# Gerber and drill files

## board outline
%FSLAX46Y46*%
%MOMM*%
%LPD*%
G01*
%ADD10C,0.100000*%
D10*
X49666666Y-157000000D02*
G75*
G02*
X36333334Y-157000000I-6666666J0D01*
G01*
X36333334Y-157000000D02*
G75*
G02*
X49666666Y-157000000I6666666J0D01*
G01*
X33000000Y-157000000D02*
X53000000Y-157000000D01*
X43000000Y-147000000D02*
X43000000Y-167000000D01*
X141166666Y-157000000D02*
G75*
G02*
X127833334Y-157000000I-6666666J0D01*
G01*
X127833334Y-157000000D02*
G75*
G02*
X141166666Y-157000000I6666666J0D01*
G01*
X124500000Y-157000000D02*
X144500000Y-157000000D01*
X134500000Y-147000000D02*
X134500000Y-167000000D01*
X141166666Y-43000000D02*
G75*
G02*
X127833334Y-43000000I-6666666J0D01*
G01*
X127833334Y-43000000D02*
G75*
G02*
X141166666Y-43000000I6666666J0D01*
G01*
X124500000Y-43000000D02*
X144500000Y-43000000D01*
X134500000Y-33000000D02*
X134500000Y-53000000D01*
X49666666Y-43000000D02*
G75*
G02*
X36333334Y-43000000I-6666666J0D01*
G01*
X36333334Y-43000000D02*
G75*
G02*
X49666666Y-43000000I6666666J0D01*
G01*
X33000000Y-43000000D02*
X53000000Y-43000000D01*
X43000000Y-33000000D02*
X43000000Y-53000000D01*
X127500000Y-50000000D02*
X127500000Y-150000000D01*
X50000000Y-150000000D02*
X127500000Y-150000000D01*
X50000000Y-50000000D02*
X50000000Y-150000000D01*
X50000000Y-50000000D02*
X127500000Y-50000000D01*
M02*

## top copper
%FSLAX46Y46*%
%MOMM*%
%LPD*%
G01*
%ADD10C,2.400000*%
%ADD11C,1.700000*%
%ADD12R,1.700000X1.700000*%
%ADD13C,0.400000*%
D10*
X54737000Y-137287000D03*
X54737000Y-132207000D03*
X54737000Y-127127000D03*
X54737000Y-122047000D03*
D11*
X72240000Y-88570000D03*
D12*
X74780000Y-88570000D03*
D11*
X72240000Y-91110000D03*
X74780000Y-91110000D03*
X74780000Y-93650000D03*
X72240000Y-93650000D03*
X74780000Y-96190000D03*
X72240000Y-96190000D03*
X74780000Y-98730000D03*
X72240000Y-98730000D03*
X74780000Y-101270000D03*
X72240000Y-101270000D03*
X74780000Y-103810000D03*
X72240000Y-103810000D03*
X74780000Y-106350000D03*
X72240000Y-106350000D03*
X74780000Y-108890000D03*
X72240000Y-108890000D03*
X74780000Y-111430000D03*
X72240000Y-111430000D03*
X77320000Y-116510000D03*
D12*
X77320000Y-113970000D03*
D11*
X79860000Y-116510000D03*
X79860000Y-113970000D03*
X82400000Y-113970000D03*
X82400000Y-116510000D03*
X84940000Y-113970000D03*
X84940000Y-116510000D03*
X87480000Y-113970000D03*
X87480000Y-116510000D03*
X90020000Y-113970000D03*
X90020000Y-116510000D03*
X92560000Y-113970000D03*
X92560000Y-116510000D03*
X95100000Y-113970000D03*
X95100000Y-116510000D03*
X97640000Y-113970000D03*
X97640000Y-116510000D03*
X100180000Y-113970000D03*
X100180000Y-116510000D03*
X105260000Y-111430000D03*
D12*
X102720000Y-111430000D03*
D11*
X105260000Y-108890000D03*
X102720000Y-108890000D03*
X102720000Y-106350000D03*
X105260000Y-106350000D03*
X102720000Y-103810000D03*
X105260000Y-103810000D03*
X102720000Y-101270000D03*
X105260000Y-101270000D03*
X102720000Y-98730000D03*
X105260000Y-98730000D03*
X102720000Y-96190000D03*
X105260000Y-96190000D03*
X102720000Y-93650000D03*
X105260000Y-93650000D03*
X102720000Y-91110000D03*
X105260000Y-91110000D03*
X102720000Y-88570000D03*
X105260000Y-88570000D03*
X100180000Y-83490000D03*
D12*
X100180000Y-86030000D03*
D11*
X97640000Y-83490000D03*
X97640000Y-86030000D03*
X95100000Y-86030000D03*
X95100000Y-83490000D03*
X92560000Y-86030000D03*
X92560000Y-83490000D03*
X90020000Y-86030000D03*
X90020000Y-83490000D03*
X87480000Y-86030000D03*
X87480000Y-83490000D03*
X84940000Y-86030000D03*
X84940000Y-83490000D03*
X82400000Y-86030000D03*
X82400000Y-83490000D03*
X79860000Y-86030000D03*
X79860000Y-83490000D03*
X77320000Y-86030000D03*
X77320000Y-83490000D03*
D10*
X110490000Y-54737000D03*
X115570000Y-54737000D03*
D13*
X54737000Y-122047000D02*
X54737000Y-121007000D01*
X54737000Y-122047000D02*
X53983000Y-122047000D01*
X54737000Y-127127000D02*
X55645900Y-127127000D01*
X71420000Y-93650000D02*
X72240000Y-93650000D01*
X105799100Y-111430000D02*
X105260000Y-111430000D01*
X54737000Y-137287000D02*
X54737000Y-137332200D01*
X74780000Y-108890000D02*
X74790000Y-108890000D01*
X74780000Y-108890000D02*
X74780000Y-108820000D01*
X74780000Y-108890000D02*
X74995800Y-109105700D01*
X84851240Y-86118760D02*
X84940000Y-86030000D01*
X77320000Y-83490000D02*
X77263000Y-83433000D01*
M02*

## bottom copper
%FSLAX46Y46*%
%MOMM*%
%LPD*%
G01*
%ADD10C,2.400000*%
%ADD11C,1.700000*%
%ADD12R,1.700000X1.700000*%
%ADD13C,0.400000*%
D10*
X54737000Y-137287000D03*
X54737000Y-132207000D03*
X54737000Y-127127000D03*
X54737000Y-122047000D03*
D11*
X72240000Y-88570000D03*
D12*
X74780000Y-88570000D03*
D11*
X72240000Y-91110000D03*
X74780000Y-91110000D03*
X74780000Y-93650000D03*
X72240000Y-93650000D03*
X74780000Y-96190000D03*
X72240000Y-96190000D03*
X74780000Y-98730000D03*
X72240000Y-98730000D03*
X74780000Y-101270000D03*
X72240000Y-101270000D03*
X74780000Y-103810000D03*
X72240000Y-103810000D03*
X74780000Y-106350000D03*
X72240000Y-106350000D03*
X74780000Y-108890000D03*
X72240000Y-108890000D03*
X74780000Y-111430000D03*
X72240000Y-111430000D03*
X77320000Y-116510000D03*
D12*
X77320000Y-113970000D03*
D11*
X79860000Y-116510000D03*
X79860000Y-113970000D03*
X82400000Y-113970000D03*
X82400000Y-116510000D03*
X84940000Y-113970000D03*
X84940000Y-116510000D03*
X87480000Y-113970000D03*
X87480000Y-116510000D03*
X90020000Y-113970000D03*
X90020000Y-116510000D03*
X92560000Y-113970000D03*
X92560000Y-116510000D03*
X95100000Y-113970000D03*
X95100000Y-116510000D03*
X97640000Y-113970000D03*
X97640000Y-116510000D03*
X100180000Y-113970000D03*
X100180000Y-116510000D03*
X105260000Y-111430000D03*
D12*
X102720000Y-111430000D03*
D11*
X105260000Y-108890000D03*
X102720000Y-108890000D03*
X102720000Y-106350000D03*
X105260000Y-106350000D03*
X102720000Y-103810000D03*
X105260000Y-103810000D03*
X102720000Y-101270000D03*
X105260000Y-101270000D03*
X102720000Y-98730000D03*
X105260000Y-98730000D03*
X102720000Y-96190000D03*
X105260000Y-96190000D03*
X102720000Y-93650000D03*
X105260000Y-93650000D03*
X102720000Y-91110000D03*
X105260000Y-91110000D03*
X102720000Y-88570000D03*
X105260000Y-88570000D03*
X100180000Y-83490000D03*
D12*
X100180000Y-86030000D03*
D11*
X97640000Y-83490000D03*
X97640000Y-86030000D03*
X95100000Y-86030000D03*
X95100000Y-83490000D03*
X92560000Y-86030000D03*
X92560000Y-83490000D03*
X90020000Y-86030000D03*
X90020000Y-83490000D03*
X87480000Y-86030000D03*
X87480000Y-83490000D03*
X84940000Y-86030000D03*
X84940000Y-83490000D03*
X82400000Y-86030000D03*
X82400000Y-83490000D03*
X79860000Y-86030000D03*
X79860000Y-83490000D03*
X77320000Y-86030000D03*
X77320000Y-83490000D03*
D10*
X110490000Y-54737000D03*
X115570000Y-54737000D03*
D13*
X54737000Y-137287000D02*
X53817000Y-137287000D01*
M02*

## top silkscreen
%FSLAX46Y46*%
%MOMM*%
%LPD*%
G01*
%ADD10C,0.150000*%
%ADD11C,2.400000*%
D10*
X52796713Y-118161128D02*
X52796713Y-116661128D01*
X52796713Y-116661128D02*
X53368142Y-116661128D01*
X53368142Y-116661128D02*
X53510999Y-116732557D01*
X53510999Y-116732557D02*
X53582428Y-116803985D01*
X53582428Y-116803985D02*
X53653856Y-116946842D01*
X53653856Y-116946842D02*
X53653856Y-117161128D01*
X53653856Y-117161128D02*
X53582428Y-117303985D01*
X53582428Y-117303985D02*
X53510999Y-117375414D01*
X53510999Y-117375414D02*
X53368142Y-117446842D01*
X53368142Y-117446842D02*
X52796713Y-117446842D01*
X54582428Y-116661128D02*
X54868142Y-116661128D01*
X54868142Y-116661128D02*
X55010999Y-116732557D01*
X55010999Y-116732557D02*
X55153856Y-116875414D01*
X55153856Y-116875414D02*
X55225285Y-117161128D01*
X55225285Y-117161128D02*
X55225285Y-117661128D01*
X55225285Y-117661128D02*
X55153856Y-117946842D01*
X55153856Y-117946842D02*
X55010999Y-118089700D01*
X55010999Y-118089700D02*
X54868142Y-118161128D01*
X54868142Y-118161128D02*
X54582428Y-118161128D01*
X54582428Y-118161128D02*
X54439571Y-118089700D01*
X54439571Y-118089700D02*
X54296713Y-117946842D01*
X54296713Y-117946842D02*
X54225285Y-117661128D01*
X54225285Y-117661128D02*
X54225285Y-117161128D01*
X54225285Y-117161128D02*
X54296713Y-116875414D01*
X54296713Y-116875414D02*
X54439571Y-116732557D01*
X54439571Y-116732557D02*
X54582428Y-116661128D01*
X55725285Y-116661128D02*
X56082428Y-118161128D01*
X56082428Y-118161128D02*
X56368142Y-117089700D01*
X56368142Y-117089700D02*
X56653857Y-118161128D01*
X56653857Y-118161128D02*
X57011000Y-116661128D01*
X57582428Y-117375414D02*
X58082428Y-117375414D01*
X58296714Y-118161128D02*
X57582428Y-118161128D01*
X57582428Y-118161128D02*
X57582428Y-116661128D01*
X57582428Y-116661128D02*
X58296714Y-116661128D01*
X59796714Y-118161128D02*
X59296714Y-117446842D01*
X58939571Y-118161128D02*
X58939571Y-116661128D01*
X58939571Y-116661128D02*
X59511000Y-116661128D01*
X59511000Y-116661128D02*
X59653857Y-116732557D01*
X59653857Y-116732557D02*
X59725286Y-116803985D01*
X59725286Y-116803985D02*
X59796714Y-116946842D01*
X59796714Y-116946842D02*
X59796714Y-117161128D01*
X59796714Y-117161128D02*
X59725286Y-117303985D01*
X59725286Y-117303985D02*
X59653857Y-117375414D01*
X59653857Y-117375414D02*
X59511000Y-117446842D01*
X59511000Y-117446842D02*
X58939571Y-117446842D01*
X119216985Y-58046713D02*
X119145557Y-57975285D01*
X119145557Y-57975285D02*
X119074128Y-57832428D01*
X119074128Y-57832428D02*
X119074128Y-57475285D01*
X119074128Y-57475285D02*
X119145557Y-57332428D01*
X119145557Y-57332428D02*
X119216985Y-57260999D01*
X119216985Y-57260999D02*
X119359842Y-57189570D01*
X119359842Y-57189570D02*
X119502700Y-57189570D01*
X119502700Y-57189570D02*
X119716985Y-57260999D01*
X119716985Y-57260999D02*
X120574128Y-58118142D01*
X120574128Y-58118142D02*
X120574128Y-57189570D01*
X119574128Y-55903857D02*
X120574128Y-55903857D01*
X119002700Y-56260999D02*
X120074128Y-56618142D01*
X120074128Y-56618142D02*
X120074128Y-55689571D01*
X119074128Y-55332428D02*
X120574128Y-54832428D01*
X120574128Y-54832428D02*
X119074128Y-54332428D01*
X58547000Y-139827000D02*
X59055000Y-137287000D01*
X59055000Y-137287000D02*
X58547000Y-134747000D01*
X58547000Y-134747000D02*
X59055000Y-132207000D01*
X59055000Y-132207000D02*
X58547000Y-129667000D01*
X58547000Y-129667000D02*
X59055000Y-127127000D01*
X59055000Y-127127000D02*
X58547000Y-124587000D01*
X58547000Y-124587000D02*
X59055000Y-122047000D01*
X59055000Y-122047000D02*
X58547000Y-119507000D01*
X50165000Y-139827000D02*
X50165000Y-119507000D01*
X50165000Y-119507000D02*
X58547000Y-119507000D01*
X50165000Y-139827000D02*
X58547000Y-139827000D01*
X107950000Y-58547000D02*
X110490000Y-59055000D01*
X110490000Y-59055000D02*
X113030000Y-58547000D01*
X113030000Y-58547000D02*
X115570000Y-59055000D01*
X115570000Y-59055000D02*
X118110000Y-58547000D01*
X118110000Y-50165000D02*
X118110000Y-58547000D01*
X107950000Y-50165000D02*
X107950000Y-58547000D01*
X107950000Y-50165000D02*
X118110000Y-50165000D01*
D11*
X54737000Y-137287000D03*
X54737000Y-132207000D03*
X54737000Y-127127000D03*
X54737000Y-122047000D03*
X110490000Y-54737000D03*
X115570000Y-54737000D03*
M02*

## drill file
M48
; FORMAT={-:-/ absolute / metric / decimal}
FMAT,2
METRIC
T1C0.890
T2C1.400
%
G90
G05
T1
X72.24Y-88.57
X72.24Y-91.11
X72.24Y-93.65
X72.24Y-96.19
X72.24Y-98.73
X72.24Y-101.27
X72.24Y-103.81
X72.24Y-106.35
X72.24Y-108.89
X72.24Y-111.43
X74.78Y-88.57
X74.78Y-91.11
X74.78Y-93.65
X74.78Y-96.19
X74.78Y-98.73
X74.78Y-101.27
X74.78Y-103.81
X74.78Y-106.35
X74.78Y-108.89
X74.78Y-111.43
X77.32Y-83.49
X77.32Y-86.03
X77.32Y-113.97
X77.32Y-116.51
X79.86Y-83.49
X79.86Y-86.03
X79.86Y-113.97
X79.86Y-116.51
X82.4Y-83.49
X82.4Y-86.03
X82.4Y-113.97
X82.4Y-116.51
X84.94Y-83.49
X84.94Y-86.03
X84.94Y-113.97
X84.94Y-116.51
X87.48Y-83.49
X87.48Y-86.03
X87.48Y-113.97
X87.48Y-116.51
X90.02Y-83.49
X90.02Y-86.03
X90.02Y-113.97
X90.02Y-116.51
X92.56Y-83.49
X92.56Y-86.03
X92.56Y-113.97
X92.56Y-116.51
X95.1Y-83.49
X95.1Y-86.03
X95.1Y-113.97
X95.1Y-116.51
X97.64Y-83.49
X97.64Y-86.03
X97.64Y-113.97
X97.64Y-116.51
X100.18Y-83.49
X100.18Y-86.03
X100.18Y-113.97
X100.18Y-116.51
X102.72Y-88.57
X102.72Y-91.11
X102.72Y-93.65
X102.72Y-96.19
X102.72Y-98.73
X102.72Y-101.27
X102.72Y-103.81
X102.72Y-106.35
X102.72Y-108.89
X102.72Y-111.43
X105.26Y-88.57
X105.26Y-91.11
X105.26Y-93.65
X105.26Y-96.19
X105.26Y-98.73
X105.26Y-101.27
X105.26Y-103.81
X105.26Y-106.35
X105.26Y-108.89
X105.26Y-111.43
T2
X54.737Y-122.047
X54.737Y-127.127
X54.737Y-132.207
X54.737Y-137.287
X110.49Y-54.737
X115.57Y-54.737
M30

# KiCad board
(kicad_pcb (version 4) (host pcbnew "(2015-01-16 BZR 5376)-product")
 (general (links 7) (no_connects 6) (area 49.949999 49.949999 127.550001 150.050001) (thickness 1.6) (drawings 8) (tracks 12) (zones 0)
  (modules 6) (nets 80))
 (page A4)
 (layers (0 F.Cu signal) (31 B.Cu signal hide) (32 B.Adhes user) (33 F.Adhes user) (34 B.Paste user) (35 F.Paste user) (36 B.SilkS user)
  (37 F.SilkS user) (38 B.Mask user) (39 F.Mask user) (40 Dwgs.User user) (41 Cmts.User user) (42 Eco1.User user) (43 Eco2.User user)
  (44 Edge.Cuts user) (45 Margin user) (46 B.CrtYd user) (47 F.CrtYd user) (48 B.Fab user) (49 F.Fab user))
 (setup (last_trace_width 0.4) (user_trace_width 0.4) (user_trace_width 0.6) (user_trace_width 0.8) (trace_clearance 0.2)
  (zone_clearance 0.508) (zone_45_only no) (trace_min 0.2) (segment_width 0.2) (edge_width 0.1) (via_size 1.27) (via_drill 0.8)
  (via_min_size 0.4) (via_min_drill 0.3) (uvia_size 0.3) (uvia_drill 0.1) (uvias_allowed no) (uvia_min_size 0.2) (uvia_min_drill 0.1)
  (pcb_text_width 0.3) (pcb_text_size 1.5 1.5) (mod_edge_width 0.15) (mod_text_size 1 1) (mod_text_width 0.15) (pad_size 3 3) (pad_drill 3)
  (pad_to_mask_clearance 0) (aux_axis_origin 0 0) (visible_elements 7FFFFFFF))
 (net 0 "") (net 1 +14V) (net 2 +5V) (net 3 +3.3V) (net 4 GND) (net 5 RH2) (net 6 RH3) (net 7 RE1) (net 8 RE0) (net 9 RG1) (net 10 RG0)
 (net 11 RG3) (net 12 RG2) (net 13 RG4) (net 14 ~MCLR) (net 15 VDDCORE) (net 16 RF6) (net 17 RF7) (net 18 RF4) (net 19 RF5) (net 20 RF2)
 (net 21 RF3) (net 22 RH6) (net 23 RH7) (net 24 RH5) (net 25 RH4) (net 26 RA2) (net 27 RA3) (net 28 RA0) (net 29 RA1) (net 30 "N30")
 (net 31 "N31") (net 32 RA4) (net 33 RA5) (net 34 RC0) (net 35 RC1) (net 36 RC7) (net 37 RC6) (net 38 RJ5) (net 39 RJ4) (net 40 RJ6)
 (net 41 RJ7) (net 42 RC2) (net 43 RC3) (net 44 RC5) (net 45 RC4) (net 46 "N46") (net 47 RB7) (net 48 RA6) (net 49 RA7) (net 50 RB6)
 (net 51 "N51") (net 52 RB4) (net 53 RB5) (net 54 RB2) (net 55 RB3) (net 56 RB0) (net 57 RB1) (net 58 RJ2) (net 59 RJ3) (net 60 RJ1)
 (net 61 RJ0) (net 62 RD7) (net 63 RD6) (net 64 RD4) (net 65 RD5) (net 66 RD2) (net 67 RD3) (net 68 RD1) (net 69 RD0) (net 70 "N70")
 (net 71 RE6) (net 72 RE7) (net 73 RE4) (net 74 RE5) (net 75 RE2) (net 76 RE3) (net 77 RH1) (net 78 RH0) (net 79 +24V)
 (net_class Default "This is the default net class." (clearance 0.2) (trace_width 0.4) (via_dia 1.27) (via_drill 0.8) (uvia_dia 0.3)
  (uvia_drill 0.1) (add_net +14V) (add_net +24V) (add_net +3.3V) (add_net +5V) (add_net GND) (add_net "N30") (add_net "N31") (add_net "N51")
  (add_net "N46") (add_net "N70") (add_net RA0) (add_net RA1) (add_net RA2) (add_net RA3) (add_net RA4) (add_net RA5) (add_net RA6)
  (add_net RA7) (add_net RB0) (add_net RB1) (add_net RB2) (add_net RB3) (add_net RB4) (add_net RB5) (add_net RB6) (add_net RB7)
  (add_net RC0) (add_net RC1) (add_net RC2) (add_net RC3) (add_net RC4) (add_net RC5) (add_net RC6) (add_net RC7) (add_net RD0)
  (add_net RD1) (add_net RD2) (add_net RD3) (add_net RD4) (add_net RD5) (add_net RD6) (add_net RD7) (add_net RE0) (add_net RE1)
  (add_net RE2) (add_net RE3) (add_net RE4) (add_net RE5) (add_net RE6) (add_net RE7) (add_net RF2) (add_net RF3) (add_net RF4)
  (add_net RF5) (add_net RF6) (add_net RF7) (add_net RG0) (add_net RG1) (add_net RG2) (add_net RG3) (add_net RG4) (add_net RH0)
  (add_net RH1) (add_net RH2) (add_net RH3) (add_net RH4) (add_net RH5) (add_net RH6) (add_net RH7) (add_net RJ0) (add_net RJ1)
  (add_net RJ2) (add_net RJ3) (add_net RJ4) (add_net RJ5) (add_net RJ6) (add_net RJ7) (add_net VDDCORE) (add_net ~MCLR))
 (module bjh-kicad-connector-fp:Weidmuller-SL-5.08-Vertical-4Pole (layer F.Cu) (at 54.737 137.287 90)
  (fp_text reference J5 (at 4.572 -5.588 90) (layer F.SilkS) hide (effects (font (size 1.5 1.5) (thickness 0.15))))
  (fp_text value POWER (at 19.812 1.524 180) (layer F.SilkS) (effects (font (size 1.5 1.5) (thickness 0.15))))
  (fp_line (start -2.54 3.81) (end 0 4.318) (layer F.SilkS) (width 0.15))
  (fp_line (start 0 4.318) (end 2.54 3.81) (layer F.SilkS) (width 0.15))
  (fp_line (start 2.54 3.81) (end 5.08 4.318) (layer F.SilkS) (width 0.15))
  (fp_line (start 5.08 4.318) (end 7.62 3.81) (layer F.SilkS) (width 0.15))
  (fp_line (start 7.62 3.81) (end 10.16 4.318) (layer F.SilkS) (width 0.15))
  (fp_line (start 10.16 4.318) (end 12.7 3.81) (layer F.SilkS) (width 0.15))
  (fp_line (start 12.7 3.81) (end 15.24 4.318) (layer F.SilkS) (width 0.15))
  (fp_line (start 15.24 4.318) (end 17.78 3.81) (layer F.SilkS) (width 0.15))
  (fp_line (start -2.54 -4.572) (end 17.78 -4.572) (layer F.SilkS) (width 0.15))
  (fp_line (start 17.78 -4.572) (end 17.78 3.81) (layer F.SilkS) (width 0.15))
  (fp_line (start -2.54 -4.572) (end -2.54 3.81) (layer F.SilkS) (width 0.15))
  (pad 1 thru_hole circle (at 0 0 90) (size 2.4 2.4) (drill 1.4) (layers *.Cu *.Mask F.SilkS) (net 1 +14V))
  (pad 2 thru_hole circle (at 5.08 0 90) (size 2.4 2.4) (drill 1.4) (layers *.Cu *.Mask F.SilkS) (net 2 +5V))
  (pad 3 thru_hole circle (at 10.16 0 90) (size 2.4 2.4) (drill 1.4) (layers *.Cu *.Mask F.SilkS) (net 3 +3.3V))
  (pad 4 thru_hole circle (at 15.24 0 90) (size 2.4 2.4) (drill 1.4) (layers *.Cu *.Mask F.SilkS) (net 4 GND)))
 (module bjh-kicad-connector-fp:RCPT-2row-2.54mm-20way (layer B.Cu) (at 73.51 88.57 270)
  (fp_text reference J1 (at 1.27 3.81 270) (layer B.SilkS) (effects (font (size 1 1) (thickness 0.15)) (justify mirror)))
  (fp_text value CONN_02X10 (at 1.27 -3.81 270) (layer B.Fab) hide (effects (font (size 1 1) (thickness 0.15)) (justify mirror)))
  (pad 2 thru_hole circle (at 0 1.27 270) (size 1.7 1.7) (drill 0.89) (layers *.Cu *.Mask B.SilkS) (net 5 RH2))
  (pad 1 thru_hole rect (at 0 -1.27 270) (size 1.7 1.7) (drill 0.89) (layers *.Cu *.Mask B.SilkS) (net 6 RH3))
  (pad 4 thru_hole circle (at 2.54 1.27 270) (size 1.7 1.7) (drill 0.89) (layers *.Cu *.Mask B.SilkS) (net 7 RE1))
  (pad 3 thru_hole circle (at 2.54 -1.27 270) (size 1.7 1.7) (drill 0.89) (layers *.Cu *.Mask B.SilkS) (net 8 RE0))
  (pad 5 thru_hole circle (at 5.08 -1.27 270) (size 1.7 1.7) (drill 0.89) (layers *.Cu *.Mask B.SilkS) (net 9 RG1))
  (pad 6 thru_hole circle (at 5.08 1.27 270) (size 1.7 1.7) (drill 0.89) (layers *.Cu *.Mask B.SilkS) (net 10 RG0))
  (pad 7 thru_hole circle (at 7.62 -1.27 270) (size 1.7 1.7) (drill 0.89) (layers *.Cu *.Mask B.SilkS) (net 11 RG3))
  (pad 8 thru_hole circle (at 7.62 1.27 270) (size 1.7 1.7) (drill 0.89) (layers *.Cu *.Mask B.SilkS) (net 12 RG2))
  (pad 9 thru_hole circle (at 10.16 -1.27 270) (size 1.7 1.7) (drill 0.89) (layers *.Cu *.Mask B.SilkS) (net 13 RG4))
  (pad 10 thru_hole circle (at 10.16 1.27 270) (size 1.7 1.7) (drill 0.89) (layers *.Cu *.Mask B.SilkS) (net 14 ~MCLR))
  (pad 11 thru_hole circle (at 12.7 -1.27 270) (size 1.7 1.7) (drill 0.89) (layers *.Cu *.Mask B.SilkS) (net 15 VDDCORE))
  (pad 12 thru_hole circle (at 12.7 1.27 270) (size 1.7 1.7) (drill 0.89) (layers *.Cu *.Mask B.SilkS) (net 4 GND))
  (pad 13 thru_hole circle (at 15.24 -1.27 270) (size 1.7 1.7) (drill 0.89) (layers *.Cu *.Mask B.SilkS) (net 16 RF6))
  (pad 14 thru_hole circle (at 15.24 1.27 270) (size 1.7 1.7) (drill 0.89) (layers *.Cu *.Mask B.SilkS) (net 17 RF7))
  (pad 15 thru_hole circle (at 17.78 -1.27 270) (size 1.7 1.7) (drill 0.89) (layers *.Cu *.Mask B.SilkS) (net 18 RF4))
  (pad 16 thru_hole circle (at 17.78 1.27 270) (size 1.7 1.7) (drill 0.89) (layers *.Cu *.Mask B.SilkS) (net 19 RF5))
  (pad 17 thru_hole circle (at 20.32 -1.27 270) (size 1.7 1.7) (drill 0.89) (layers *.Cu *.Mask B.SilkS) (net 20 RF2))
  (pad 18 thru_hole circle (at 20.32 1.27 270) (size 1.7 1.7) (drill 0.89) (layers *.Cu *.Mask B.SilkS) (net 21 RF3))
  (pad 19 thru_hole circle (at 22.86 -1.27 270) (size 1.7 1.7) (drill 0.89) (layers *.Cu *.Mask B.SilkS) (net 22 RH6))
  (pad 20 thru_hole circle (at 22.86 1.27 270) (size 1.7 1.7) (drill 0.89) (layers *.Cu *.Mask B.SilkS) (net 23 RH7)))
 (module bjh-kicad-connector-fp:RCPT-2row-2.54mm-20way (layer B.Cu) (at 77.32 115.24)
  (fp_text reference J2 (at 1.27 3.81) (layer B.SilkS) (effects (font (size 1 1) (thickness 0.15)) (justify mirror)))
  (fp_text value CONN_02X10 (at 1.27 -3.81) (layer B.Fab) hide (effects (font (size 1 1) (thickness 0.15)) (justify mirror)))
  (pad 2 thru_hole circle (at 0 1.27) (size 1.7 1.7) (drill 0.89) (layers *.Cu *.Mask B.SilkS) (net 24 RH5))
  (pad 1 thru_hole rect (at 0 -1.27) (size 1.7 1.7) (drill 0.89) (layers *.Cu *.Mask B.SilkS) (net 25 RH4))
  (pad 4 thru_hole circle (at 2.54 1.27) (size 1.7 1.7) (drill 0.89) (layers *.Cu *.Mask B.SilkS) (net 3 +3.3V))
  (pad 3 thru_hole circle (at 2.54 -1.27) (size 1.7 1.7) (drill 0.89) (layers *.Cu *.Mask B.SilkS) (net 4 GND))
  (pad 5 thru_hole circle (at 5.08 -1.27) (size 1.7 1.7) (drill 0.89) (layers *.Cu *.Mask B.SilkS) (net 4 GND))
  (pad 6 thru_hole circle (at 5.08 1.27) (size 1.7 1.7) (drill 0.89) (layers *.Cu *.Mask B.SilkS) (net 3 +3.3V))
  (pad 7 thru_hole circle (at 7.62 -1.27) (size 1.7 1.7) (drill 0.89) (layers *.Cu *.Mask B.SilkS) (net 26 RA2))
  (pad 8 thru_hole circle (at 7.62 1.27) (size 1.7 1.7) (drill 0.89) (layers *.Cu *.Mask B.SilkS) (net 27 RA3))
  (pad 9 thru_hole circle (at 10.16 -1.27) (size 1.7 1.7) (drill 0.89) (layers *.Cu *.Mask B.SilkS) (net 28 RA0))
  (pad 10 thru_hole circle (at 10.16 1.27) (size 1.7 1.7) (drill 0.89) (layers *.Cu *.Mask B.SilkS) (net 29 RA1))
  (pad 11 thru_hole circle (at 12.7 -1.27) (size 1.7 1.7) (drill 0.89) (layers *.Cu *.Mask B.SilkS) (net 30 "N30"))
  (pad 12 thru_hole circle (at 12.7 1.27) (size 1.7 1.7) (drill 0.89) (layers *.Cu *.Mask B.SilkS) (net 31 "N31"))
  (pad 13 thru_hole circle (at 15.24 -1.27) (size 1.7 1.7) (drill 0.89) (layers *.Cu *.Mask B.SilkS) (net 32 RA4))
  (pad 14 thru_hole circle (at 15.24 1.27) (size 1.7 1.7) (drill 0.89) (layers *.Cu *.Mask B.SilkS) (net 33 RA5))
  (pad 15 thru_hole circle (at 17.78 -1.27) (size 1.7 1.7) (drill 0.89) (layers *.Cu *.Mask B.SilkS) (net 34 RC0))
  (pad 16 thru_hole circle (at 17.78 1.27) (size 1.7 1.7) (drill 0.89) (layers *.Cu *.Mask B.SilkS) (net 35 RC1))
  (pad 17 thru_hole circle (at 20.32 -1.27) (size 1.7 1.7) (drill 0.89) (layers *.Cu *.Mask B.SilkS) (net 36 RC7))
  (pad 18 thru_hole circle (at 20.32 1.27) (size 1.7 1.7) (drill 0.89) (layers *.Cu *.Mask B.SilkS) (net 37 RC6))
  (pad 19 thru_hole circle (at 22.86 -1.27) (size 1.7 1.7) (drill 0.89) (layers *.Cu *.Mask B.SilkS) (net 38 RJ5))
  (pad 20 thru_hole circle (at 22.86 1.27) (size 1.7 1.7) (drill 0.89) (layers *.Cu *.Mask B.SilkS) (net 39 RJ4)))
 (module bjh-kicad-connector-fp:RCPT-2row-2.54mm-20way (layer B.Cu) (at 103.99 111.43 90)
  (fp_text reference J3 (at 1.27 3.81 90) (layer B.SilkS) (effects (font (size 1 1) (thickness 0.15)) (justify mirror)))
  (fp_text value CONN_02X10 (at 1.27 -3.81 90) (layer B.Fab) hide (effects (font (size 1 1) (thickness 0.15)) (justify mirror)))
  (pad 2 thru_hole circle (at 0 1.27 90) (size 1.7 1.7) (drill 0.89) (layers *.Cu *.Mask B.SilkS) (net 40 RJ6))
  (pad 1 thru_hole rect (at 0 -1.27 90) (size 1.7 1.7) (drill 0.89) (layers *.Cu *.Mask B.SilkS) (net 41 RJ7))
  (pad 4 thru_hole circle (at 2.54 1.27 90) (size 1.7 1.7) (drill 0.89) (layers *.Cu *.Mask B.SilkS) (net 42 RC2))
  (pad 3 thru_hole circle (at 2.54 -1.27 90) (size 1.7 1.7) (drill 0.89) (layers *.Cu *.Mask B.SilkS) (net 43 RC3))
  (pad 5 thru_hole circle (at 5.08 -1.27 90) (size 1.7 1.7) (drill 0.89) (layers *.Cu *.Mask B.SilkS) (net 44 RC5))
  (pad 6 thru_hole circle (at 5.08 1.27 90) (size 1.7 1.7) (drill 0.89) (layers *.Cu *.Mask B.SilkS) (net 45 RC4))
  (pad 7 thru_hole circle (at 7.62 -1.27 90) (size 1.7 1.7) (drill 0.89) (layers *.Cu *.Mask B.SilkS) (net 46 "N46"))
  (pad 8 thru_hole circle (at 7.62 1.27 90) (size 1.7 1.7) (drill 0.89) (layers *.Cu *.Mask B.SilkS) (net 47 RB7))
  (pad 9 thru_hole circle (at 10.16 -1.27 90) (size 1.7 1.7) (drill 0.89) (layers *.Cu *.Mask B.SilkS) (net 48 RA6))
  (pad 10 thru_hole circle (at 10.16 1.27 90) (size 1.7 1.7) (drill 0.89) (layers *.Cu *.Mask B.SilkS) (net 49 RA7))
  (pad 11 thru_hole circle (at 12.7 -1.27 90) (size 1.7 1.7) (drill 0.89) (layers *.Cu *.Mask B.SilkS) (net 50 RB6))
  (pad 12 thru_hole circle (at 12.7 1.27 90) (size 1.7 1.7) (drill 0.89) (layers *.Cu *.Mask B.SilkS) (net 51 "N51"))
  (pad 13 thru_hole circle (at 15.24 -1.27 90) (size 1.7 1.7) (drill 0.89) (layers *.Cu *.Mask B.SilkS) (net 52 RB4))
  (pad 14 thru_hole circle (at 15.24 1.27 90) (size 1.7 1.7) (drill 0.89) (layers *.Cu *.Mask B.SilkS) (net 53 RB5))
  (pad 15 thru_hole circle (at 17.78 -1.27 90) (size 1.7 1.7) (drill 0.89) (layers *.Cu *.Mask B.SilkS) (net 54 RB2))
  (pad 16 thru_hole circle (at 17.78 1.27 90) (size 1.7 1.7) (drill 0.89) (layers *.Cu *.Mask B.SilkS) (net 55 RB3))
  (pad 17 thru_hole circle (at 20.32 -1.27 90) (size 1.7 1.7) (drill 0.89) (layers *.Cu *.Mask B.SilkS) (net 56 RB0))
  (pad 18 thru_hole circle (at 20.32 1.27 90) (size 1.7 1.7) (drill 0.89) (layers *.Cu *.Mask B.SilkS) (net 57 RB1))
  (pad 19 thru_hole circle (at 22.86 -1.27 90) (size 1.7 1.7) (drill 0.89) (layers *.Cu *.Mask B.SilkS) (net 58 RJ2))
  (pad 20 thru_hole circle (at 22.86 1.27 90) (size 1.7 1.7) (drill 0.89) (layers *.Cu *.Mask B.SilkS) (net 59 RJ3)))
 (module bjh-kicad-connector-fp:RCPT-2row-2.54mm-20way (layer B.Cu) (at 100.18 84.76 180)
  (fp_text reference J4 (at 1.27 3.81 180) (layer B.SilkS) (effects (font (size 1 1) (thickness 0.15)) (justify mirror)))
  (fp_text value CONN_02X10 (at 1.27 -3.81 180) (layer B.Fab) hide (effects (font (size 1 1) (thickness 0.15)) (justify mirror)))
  (pad 2 thru_hole circle (at 0 1.27 180) (size 1.7 1.7) (drill 0.89) (layers *.Cu *.Mask B.SilkS) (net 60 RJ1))
  (pad 1 thru_hole rect (at 0 -1.27 180) (size 1.7 1.7) (drill 0.89) (layers *.Cu *.Mask B.SilkS) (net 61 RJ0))
  (pad 4 thru_hole circle (at 2.54 1.27 180) (size 1.7 1.7) (drill 0.89) (layers *.Cu *.Mask B.SilkS) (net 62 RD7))
  (pad 3 thru_hole circle (at 2.54 -1.27 180) (size 1.7 1.7) (drill 0.89) (layers *.Cu *.Mask B.SilkS) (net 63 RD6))
  (pad 5 thru_hole circle (at 5.08 -1.27 180) (size 1.7 1.7) (drill 0.89) (layers *.Cu *.Mask B.SilkS) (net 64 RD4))
  (pad 6 thru_hole circle (at 5.08 1.27 180) (size 1.7 1.7) (drill 0.89) (layers *.Cu *.Mask B.SilkS) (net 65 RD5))
  (pad 7 thru_hole circle (at 7.62 -1.27 180) (size 1.7 1.7) (drill 0.89) (layers *.Cu *.Mask B.SilkS) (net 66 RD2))
  (pad 8 thru_hole circle (at 7.62 1.27 180) (size 1.7 1.7) (drill 0.89) (layers *.Cu *.Mask B.SilkS) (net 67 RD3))
  (pad 9 thru_hole circle (at 10.16 -1.27 180) (size 1.7 1.7) (drill 0.89) (layers *.Cu *.Mask B.SilkS) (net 4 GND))
  (pad 10 thru_hole circle (at 10.16 1.27 180) (size 1.7 1.7) (drill 0.89) (layers *.Cu *.Mask B.SilkS) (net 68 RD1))
  (pad 11 thru_hole circle (at 12.7 -1.27 180) (size 1.7 1.7) (drill 0.89) (layers *.Cu *.Mask B.SilkS) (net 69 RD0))
  (pad 12 thru_hole circle (at 12.7 1.27 180) (size 1.7 1.7) (drill 0.89) (layers *.Cu *.Mask B.SilkS) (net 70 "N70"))
  (pad 13 thru_hole circle (at 15.24 -1.27 180) (size 1.7 1.7) (drill 0.89) (layers *.Cu *.Mask B.SilkS) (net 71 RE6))
  (pad 14 thru_hole circle (at 15.24 1.27 180) (size 1.7 1.7) (drill 0.89) (layers *.Cu *.Mask B.SilkS) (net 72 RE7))
  (pad 15 thru_hole circle (at 17.78 -1.27 180) (size 1.7 1.7) (drill 0.89) (layers *.Cu *.Mask B.SilkS) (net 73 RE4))
  (pad 16 thru_hole circle (at 17.78 1.27 180) (size 1.7 1.7) (drill 0.89) (layers *.Cu *.Mask B.SilkS) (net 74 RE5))
  (pad 17 thru_hole circle (at 20.32 -1.27 180) (size 1.7 1.7) (drill 0.89) (layers *.Cu *.Mask B.SilkS) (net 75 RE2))
  (pad 18 thru_hole circle (at 20.32 1.27 180) (size 1.7 1.7) (drill 0.89) (layers *.Cu *.Mask B.SilkS) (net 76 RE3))
  (pad 19 thru_hole circle (at 22.86 -1.27 180) (size 1.7 1.7) (drill 0.89) (layers *.Cu *.Mask B.SilkS) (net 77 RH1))
  (pad 20 thru_hole circle (at 22.86 1.27 180) (size 1.7 1.7) (drill 0.89) (layers *.Cu *.Mask B.SilkS) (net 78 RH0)))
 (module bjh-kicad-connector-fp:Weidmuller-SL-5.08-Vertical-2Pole (layer F.Cu) (at 110.49 54.737)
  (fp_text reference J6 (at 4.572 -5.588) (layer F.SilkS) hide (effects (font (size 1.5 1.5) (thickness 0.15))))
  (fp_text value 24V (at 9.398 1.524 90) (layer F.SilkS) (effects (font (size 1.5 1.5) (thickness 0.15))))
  (fp_line (start -2.54 3.81) (end 0 4.318) (layer F.SilkS) (width 0.15))
  (fp_line (start 0 4.318) (end 2.54 3.81) (layer F.SilkS) (width 0.15))
  (fp_line (start 2.54 3.81) (end 5.08 4.318) (layer F.SilkS) (width 0.15))
  (fp_line (start 5.08 4.318) (end 7.62 3.81) (layer F.SilkS) (width 0.15))
  (fp_line (start 7.62 -4.572) (end 7.62 3.81) (layer F.SilkS) (width 0.15))
  (fp_line (start -2.54 -4.572) (end -2.54 3.81) (layer F.SilkS) (width 0.15))
  (fp_line (start -2.54 -4.572) (end 7.62 -4.572) (layer F.SilkS) (width 0.15))
  (pad 1 thru_hole circle (at 0 0) (size 2.4 2.4) (drill 1.4) (layers *.Cu *.Mask F.SilkS) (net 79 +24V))
  (pad 2 thru_hole circle (at 5.08 0) (size 2.4 2.4) (drill 1.4) (layers *.Cu *.Mask F.SilkS) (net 4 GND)))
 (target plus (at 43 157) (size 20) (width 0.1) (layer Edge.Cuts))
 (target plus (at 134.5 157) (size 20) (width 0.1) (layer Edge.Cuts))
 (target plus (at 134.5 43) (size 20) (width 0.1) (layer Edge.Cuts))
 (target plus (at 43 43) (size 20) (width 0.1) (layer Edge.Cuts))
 (gr_line (start 127.5 50) (end 127.5 150) (angle 90) (layer Edge.Cuts) (width 0.1))
 (gr_line (start 50 150) (end 127.5 150) (angle 90) (layer Edge.Cuts) (width 0.1))
 (gr_line (start 50 50) (end 50 150) (angle 90) (layer Edge.Cuts) (width 0.1))
 (gr_line (start 50 50) (end 127.5 50) (angle 90) (layer Edge.Cuts) (width 0.1))
 (segment (start 54.737 122.047) (end 54.737 121.007) (width 0.4) (layer F.Cu) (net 4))
 (segment (start 54.737 122.047) (end 53.983 122.047) (width 0.4) (layer F.Cu) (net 4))
 (segment (start 54.737 127.127) (end 55.6459 127.127) (width 0.4) (layer F.Cu) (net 3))
 (segment (start 71.42 93.65) (end 72.24 93.65) (width 0.4) (layer F.Cu) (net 10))
 (segment (start 105.7991 111.43) (end 105.26 111.43) (width 0.4) (layer F.Cu) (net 40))
 (segment (start 54.737 137.287) (end 53.817 137.287) (width 0.4) (layer B.Cu) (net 1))
 (segment (start 54.737 137.287) (end 54.737 137.3322) (width 0.4) (layer F.Cu) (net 1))
 (segment (start 74.78 108.89) (end 74.79 108.89) (width 0.4) (layer F.Cu) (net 20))
 (segment (start 74.78 108.89) (end 74.78 108.82) (width 0.4) (layer F.Cu) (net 20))
 (segment (start 74.78 108.89) (end 74.9958 109.1057) (width 0.4) (layer F.Cu) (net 20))
 (segment (start 84.85124 86.11876) (end 84.94 86.03) (width 0.4) (layer F.Cu) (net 71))
 (segment (start 77.32 83.49) (end 77.263 83.433) (width 0.4) (layer F.Cu) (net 78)))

